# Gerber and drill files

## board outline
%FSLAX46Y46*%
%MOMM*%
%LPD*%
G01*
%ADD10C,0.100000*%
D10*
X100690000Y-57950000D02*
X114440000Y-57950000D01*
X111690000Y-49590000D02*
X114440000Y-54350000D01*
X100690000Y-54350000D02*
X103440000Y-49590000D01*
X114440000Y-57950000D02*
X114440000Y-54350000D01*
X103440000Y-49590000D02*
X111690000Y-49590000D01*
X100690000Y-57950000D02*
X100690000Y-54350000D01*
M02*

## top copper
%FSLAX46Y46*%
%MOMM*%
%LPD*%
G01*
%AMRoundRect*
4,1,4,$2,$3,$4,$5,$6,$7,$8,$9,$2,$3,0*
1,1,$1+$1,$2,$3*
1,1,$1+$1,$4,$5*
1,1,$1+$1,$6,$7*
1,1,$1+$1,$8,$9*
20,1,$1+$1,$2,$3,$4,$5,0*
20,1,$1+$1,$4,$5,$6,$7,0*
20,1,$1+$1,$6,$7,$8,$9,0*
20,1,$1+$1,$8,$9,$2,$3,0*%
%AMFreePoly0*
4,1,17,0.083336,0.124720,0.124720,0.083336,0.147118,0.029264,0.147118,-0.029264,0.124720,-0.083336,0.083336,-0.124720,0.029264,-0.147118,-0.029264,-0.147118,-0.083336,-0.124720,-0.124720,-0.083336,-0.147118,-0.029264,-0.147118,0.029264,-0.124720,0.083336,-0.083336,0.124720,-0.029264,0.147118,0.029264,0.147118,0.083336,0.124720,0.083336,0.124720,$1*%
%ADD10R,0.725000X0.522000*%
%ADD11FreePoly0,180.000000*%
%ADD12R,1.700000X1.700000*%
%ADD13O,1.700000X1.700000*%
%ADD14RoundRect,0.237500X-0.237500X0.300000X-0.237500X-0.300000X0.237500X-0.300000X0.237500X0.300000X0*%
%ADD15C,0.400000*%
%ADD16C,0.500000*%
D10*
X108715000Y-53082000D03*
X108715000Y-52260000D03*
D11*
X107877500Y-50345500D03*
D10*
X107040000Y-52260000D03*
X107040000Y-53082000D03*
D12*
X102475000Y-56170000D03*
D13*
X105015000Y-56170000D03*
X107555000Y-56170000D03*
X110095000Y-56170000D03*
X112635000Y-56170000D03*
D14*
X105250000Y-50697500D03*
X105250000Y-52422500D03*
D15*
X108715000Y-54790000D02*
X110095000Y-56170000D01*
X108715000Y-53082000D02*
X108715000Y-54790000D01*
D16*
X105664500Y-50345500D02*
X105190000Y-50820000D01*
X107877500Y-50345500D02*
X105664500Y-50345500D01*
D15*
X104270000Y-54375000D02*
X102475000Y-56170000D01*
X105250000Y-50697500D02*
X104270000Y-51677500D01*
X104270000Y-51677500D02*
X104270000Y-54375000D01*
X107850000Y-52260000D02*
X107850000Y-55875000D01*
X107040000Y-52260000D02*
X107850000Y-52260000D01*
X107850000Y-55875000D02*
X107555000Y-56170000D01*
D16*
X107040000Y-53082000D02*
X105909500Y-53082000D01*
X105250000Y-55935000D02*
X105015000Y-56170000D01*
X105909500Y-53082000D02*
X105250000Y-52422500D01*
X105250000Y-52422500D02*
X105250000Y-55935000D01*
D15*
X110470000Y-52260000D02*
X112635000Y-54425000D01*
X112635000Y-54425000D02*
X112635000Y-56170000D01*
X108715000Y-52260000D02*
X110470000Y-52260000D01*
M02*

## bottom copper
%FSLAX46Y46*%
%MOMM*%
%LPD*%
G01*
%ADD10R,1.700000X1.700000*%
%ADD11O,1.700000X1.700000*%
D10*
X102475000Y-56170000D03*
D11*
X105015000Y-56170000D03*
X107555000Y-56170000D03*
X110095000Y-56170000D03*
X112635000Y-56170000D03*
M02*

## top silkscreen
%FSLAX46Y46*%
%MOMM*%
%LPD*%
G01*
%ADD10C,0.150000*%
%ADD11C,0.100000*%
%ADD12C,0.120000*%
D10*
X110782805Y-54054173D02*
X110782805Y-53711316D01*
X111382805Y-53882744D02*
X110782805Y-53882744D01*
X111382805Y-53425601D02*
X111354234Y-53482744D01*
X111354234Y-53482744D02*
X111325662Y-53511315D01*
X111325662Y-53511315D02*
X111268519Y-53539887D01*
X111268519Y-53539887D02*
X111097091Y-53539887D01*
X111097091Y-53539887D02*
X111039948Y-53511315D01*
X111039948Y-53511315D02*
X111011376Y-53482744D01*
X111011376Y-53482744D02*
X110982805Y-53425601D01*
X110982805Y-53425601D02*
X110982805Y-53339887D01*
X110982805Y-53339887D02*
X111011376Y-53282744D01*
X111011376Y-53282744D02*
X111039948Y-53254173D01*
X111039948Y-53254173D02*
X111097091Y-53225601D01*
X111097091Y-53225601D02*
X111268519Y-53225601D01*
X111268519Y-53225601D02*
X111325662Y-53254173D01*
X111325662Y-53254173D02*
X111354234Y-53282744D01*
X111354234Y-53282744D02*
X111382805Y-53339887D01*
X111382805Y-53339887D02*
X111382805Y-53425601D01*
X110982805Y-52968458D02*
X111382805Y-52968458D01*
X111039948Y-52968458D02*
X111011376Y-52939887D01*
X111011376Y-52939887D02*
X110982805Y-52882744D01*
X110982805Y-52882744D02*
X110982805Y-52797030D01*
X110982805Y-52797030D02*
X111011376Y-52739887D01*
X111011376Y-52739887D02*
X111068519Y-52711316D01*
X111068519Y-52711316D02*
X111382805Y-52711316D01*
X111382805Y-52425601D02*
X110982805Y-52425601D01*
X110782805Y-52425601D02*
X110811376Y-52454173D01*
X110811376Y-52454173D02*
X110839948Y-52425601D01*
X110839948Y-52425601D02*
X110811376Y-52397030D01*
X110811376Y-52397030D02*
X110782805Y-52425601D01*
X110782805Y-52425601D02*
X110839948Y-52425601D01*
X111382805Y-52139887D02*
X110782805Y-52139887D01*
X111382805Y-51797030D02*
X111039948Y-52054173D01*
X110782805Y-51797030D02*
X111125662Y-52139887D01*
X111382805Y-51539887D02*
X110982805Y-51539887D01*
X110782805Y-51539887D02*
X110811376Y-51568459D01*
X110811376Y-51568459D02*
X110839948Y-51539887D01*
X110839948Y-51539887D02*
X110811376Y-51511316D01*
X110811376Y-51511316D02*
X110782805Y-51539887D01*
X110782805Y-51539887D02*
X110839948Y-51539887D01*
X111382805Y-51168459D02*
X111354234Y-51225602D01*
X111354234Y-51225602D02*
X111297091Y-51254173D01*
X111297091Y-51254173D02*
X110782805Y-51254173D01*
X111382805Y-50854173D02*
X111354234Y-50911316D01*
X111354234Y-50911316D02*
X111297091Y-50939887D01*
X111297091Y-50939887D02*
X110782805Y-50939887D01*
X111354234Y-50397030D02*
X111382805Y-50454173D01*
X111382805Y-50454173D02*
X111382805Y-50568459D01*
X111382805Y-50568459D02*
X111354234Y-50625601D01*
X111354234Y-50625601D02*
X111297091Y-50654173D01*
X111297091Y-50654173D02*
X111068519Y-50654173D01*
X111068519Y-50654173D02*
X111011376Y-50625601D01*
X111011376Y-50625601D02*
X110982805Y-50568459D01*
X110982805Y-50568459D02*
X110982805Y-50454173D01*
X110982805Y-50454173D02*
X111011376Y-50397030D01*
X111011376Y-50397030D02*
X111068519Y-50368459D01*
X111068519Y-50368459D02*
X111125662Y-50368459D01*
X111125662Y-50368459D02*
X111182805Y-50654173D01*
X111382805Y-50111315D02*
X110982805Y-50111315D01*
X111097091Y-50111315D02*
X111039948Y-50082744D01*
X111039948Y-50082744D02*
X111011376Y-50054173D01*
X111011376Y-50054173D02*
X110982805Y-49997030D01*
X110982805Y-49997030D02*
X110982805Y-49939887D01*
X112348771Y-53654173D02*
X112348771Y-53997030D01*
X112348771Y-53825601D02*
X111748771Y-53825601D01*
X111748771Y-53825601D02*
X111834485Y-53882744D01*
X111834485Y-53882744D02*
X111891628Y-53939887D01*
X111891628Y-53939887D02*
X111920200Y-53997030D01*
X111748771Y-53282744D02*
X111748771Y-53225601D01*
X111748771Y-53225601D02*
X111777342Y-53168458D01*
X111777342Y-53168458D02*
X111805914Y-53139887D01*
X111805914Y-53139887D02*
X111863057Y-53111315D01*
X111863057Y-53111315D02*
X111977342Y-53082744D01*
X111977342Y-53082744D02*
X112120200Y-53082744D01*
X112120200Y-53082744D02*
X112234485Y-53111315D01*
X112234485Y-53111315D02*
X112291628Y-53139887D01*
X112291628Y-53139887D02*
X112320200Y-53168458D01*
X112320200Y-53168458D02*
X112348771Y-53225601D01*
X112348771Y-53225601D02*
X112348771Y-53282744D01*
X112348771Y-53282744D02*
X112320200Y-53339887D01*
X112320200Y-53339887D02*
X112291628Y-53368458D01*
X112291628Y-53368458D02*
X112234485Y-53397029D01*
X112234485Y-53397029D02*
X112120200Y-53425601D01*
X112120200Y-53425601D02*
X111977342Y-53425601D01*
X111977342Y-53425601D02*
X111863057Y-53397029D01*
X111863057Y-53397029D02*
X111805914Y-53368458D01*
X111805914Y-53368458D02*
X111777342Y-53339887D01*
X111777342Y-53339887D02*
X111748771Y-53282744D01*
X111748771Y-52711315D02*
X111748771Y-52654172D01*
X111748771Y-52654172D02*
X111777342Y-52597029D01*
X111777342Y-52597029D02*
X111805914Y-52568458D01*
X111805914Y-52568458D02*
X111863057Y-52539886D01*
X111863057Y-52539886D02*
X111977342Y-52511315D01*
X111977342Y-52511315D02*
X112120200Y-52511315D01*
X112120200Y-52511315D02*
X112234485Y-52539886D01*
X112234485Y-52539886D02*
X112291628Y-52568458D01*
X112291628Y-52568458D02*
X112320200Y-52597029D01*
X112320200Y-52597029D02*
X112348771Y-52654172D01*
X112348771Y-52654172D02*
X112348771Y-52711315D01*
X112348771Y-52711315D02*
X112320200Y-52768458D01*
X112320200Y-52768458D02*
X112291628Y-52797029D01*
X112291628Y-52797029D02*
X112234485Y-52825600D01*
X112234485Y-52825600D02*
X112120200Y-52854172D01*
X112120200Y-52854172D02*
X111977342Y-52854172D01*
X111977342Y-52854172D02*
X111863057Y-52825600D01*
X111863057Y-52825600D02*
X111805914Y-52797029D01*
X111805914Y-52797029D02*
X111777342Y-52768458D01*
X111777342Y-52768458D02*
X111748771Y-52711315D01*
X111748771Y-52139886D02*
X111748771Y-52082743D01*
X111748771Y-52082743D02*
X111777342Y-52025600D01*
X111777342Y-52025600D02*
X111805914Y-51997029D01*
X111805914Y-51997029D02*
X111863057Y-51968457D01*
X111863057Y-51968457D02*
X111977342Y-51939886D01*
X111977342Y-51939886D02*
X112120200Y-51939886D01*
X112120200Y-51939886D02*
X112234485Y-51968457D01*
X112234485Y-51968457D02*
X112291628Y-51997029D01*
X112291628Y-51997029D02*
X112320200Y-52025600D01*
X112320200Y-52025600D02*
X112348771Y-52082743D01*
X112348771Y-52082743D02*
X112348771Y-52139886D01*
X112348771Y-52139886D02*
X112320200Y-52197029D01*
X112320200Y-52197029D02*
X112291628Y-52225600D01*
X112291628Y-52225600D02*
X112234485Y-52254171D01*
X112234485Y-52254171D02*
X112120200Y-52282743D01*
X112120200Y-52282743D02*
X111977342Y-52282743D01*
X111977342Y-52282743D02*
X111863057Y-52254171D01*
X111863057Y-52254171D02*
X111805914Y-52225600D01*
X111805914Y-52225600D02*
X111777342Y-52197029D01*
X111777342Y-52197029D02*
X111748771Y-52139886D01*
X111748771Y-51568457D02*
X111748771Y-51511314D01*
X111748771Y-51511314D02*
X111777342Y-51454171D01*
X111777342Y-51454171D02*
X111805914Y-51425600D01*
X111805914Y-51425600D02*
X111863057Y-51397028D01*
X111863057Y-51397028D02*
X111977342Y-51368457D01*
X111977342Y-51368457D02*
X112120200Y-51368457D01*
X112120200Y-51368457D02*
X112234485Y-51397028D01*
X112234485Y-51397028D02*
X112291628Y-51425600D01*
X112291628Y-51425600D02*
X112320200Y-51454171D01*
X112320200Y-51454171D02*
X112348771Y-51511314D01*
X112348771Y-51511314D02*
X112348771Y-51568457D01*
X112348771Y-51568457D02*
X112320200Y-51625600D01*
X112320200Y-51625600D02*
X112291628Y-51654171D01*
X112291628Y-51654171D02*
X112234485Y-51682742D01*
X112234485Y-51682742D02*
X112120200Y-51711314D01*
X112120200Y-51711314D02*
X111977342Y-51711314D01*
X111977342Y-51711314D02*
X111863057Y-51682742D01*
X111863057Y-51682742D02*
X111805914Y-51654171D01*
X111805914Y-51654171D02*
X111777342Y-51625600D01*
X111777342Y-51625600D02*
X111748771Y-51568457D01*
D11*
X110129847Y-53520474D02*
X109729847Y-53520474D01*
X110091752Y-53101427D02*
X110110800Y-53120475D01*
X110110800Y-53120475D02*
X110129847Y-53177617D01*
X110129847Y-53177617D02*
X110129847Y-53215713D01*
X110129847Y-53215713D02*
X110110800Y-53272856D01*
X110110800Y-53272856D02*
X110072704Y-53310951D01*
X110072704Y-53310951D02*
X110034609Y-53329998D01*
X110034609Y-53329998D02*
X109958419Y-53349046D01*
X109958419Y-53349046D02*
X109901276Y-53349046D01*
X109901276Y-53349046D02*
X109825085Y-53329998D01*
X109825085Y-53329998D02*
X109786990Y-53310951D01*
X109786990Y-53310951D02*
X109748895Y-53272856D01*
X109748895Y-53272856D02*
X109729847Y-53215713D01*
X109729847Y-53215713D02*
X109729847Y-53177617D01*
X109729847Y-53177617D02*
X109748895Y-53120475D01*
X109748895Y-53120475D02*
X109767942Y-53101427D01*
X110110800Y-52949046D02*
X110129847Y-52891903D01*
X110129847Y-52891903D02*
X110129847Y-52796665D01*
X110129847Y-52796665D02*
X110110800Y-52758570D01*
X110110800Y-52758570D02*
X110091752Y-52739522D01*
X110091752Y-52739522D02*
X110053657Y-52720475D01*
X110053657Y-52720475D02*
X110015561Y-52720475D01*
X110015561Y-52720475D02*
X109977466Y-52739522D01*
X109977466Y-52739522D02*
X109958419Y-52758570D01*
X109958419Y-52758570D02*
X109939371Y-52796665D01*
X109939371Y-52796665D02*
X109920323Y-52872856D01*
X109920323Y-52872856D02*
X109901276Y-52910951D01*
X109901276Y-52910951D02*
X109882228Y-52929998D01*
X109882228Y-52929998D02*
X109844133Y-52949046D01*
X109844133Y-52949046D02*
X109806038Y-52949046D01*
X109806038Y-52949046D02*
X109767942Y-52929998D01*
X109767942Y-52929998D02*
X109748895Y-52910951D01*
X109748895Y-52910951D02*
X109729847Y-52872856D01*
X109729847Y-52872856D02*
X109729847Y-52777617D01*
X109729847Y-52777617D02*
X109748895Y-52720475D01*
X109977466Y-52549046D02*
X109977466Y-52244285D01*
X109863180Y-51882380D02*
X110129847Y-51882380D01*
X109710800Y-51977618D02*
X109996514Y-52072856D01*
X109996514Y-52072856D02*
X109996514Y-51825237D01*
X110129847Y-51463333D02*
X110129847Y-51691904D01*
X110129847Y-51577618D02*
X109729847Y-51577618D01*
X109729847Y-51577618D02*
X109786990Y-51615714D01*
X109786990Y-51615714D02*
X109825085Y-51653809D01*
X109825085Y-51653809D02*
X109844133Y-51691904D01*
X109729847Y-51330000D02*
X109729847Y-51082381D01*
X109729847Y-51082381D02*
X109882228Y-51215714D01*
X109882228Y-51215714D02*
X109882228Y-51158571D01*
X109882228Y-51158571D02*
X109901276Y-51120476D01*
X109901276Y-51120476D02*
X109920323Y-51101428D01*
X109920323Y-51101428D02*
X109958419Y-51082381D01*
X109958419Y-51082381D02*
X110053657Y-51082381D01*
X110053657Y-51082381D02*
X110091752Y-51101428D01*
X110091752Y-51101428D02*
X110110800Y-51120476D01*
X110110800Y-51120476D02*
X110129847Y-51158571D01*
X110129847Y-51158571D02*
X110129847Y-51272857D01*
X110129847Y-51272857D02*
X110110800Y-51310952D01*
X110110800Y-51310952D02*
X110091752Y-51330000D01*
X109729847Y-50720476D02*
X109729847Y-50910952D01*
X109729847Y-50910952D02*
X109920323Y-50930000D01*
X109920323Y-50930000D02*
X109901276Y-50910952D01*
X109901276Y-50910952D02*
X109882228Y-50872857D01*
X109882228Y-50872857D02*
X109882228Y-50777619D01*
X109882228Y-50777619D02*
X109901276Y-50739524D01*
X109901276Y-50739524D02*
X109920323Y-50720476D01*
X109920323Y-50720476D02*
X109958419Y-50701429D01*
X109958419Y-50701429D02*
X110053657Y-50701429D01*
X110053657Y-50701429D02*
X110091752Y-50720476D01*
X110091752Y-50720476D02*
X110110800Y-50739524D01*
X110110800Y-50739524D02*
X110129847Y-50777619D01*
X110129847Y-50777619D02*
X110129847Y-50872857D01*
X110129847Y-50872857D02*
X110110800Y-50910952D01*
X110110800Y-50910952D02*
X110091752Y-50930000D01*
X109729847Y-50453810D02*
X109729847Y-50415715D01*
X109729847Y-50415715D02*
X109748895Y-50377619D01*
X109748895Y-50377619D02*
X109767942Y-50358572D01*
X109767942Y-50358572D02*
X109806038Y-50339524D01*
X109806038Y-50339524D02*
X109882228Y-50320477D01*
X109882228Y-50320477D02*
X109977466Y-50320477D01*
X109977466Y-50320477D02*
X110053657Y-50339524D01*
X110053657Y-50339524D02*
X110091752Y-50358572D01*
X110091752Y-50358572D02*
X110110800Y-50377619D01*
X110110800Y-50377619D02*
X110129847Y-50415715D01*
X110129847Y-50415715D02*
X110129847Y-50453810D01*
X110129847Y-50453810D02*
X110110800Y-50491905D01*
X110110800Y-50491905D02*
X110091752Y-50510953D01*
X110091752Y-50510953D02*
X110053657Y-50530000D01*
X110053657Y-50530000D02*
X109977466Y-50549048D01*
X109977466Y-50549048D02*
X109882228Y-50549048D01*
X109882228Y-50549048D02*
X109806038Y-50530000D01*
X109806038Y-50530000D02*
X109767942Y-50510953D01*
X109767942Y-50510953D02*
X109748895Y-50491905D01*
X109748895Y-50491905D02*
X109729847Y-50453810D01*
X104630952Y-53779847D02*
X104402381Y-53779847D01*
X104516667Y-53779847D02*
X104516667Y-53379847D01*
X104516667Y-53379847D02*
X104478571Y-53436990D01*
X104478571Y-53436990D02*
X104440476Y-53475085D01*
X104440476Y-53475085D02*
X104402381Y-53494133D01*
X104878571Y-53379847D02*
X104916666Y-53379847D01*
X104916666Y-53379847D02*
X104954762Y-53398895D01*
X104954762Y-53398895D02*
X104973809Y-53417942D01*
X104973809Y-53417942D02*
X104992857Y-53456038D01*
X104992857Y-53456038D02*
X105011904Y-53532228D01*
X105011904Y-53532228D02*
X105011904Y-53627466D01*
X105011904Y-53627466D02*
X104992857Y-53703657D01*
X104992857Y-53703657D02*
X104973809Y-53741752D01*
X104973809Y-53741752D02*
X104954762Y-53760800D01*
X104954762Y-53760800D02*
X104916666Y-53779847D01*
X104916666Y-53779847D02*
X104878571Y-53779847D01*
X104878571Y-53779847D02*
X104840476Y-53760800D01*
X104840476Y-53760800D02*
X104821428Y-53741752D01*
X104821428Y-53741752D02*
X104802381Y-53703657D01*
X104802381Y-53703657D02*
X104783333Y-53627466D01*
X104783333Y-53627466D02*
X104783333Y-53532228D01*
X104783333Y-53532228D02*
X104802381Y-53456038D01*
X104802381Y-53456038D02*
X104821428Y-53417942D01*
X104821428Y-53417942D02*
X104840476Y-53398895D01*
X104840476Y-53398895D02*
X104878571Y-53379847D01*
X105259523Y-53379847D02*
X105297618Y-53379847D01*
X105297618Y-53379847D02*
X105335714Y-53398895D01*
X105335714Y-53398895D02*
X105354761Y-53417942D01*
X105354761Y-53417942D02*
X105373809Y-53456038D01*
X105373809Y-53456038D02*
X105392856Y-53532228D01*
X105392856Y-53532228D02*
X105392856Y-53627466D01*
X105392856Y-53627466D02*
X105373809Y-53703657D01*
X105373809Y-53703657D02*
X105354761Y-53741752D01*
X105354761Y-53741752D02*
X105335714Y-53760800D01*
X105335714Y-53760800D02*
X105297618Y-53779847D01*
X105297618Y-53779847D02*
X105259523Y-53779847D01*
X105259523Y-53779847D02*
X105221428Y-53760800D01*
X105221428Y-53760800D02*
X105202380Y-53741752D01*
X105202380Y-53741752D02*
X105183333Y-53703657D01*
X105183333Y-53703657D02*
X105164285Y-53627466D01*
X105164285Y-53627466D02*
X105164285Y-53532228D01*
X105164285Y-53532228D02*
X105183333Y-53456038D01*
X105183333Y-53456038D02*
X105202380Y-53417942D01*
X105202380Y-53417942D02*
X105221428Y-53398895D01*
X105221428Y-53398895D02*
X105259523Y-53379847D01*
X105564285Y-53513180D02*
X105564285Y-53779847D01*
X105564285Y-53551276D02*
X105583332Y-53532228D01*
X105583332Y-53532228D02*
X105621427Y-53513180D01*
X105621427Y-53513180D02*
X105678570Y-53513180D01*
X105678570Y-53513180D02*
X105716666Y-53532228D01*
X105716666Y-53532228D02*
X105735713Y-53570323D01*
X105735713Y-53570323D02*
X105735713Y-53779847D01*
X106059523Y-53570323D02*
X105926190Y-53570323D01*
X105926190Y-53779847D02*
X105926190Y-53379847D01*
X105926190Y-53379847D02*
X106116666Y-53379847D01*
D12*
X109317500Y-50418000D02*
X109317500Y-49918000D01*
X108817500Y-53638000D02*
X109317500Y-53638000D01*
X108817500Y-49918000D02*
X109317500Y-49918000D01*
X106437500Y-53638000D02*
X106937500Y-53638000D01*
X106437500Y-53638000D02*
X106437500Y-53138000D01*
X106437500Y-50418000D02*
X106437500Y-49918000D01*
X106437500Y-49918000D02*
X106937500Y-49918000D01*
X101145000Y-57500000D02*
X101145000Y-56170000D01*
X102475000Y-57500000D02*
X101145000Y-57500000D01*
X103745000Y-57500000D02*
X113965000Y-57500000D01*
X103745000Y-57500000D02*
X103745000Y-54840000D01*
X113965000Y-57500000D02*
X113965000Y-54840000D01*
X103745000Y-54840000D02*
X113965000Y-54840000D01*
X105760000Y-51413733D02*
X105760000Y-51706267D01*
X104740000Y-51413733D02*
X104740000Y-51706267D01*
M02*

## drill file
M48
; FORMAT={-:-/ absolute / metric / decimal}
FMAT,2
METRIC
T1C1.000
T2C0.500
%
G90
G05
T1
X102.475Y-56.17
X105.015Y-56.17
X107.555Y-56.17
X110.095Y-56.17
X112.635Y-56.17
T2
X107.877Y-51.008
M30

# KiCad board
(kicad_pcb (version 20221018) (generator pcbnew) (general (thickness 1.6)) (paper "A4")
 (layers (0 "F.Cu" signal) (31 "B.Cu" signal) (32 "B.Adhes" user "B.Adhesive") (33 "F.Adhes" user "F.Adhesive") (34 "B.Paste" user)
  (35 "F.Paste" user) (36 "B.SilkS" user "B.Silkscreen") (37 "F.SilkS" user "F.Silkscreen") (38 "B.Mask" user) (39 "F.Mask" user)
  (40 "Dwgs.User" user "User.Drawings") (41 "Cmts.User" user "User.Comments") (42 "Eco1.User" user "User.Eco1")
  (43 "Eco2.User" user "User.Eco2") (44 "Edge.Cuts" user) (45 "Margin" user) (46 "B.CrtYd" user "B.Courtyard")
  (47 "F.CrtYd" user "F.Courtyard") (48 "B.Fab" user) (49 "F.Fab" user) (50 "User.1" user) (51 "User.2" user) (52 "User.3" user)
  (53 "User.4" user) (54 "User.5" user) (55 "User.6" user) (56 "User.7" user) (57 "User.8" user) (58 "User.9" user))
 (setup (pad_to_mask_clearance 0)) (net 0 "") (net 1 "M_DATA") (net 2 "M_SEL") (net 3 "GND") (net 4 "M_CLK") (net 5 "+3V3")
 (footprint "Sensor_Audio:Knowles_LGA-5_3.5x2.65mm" (layer "F.Cu") (at 107.8775 51.778 180)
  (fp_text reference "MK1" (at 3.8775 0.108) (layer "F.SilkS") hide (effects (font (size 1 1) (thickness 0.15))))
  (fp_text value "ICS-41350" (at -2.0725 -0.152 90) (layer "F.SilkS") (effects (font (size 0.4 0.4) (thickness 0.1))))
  (fp_line (start -1.44 1.36) (end -1.44 1.86) (stroke (width 0.12) (type solid)) (layer "F.SilkS"))
  (fp_line (start -0.94 -1.86) (end -1.44 -1.86) (stroke (width 0.12) (type solid)) (layer "F.SilkS"))
  (fp_line (start -0.94 1.86) (end -1.44 1.86) (stroke (width 0.12) (type solid)) (layer "F.SilkS"))
  (fp_line (start 1.44 -1.86) (end 0.94 -1.86) (stroke (width 0.12) (type solid)) (layer "F.SilkS"))
  (fp_line (start 1.44 -1.86) (end 1.44 -1.36) (stroke (width 0.12) (type solid)) (layer "F.SilkS"))
  (fp_line (start 1.44 1.36) (end 1.44 1.86) (stroke (width 0.12) (type solid)) (layer "F.SilkS"))
  (fp_line (start 1.44 1.86) (end 0.94 1.86) (stroke (width 0.12) (type solid)) (layer "F.SilkS"))
  (pad "" np_thru_hole circle (at 0 0.77 180) (size 0.5 0.5) (drill 0.5) (layers "F&B.Cu" "*.Mask"))
  (pad "1" smd rect (at -0.8375 -1.304 180) (size 0.725 0.522) (layers "F.Cu" "F.Paste" "F.Mask") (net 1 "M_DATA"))
  (pad "2" smd rect (at -0.8375 -0.482 180) (size 0.725 0.522) (layers "F.Cu" "F.Paste" "F.Mask") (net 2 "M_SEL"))
  (pad "3" smd custom (at 0 1.4325 180) (size 0.3 0.3) (layers "F.Cu" "F.Mask") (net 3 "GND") (zone_connect 0) (thermal_bridge_angle 90)
   (options (clearance outline) (anchor circle)) (primitives))
  (pad "4" smd rect (at 0.8375 -0.482 180) (size 0.725 0.522) (layers "F.Cu" "F.Paste" "F.Mask") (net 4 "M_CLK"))
  (pad "5" smd rect (at 0.8375 -1.304 180) (size 0.725 0.522) (layers "F.Cu" "F.Paste" "F.Mask") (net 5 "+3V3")))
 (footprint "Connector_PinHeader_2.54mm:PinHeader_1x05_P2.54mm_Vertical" (layer "F.Cu") (at 102.475 56.17 90)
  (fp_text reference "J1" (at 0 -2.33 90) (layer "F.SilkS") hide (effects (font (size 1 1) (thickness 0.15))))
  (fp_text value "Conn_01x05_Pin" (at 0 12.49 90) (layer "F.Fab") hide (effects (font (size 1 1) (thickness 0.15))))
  (fp_line (start -1.33 -1.33) (end 0 -1.33) (stroke (width 0.12) (type solid)) (layer "F.SilkS"))
  (fp_line (start -1.33 0) (end -1.33 -1.33) (stroke (width 0.12) (type solid)) (layer "F.SilkS"))
  (fp_line (start -1.33 1.27) (end -1.33 11.49) (stroke (width 0.12) (type solid)) (layer "F.SilkS"))
  (fp_line (start -1.33 1.27) (end 1.33 1.27) (stroke (width 0.12) (type solid)) (layer "F.SilkS"))
  (fp_line (start -1.33 11.49) (end 1.33 11.49) (stroke (width 0.12) (type solid)) (layer "F.SilkS"))
  (fp_line (start 1.33 1.27) (end 1.33 11.49) (stroke (width 0.12) (type solid)) (layer "F.SilkS"))
  (pad "1" thru_hole rect (at 0 0 90) (size 1.7 1.7) (drill 1) (layers "*.Cu" "*.Mask") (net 3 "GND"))
  (pad "2" thru_hole oval (at 0 2.54 90) (size 1.7 1.7) (drill 1) (layers "*.Cu" "*.Mask") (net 5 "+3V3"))
  (pad "3" thru_hole oval (at 0 5.08 90) (size 1.7 1.7) (drill 1) (layers "*.Cu" "*.Mask") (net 4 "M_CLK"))
  (pad "4" thru_hole oval (at 0 7.62 90) (size 1.7 1.7) (drill 1) (layers "*.Cu" "*.Mask") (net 1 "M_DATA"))
  (pad "5" thru_hole oval (at 0 10.16 90) (size 1.7 1.7) (drill 1) (layers "*.Cu" "*.Mask") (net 2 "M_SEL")))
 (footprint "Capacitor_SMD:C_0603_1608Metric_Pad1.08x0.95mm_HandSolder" (layer "F.Cu") (at 105.25 51.56 -90)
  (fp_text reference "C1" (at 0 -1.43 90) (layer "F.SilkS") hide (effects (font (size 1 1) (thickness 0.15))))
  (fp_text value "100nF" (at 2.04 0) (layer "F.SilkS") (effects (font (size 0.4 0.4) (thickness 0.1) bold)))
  (fp_line (start -0.146267 -0.51) (end 0.146267 -0.51) (stroke (width 0.12) (type solid)) (layer "F.SilkS"))
  (fp_line (start -0.146267 0.51) (end 0.146267 0.51) (stroke (width 0.12) (type solid)) (layer "F.SilkS"))
  (pad "1" smd roundrect (at -0.8625 0 270) (size 1.075 0.95) (layers "F.Cu" "F.Paste" "F.Mask") (roundrect_rratio 0.25) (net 3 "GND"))
  (pad "2" smd roundrect (at 0.8625 0 270) (size 1.075 0.95) (layers "F.Cu" "F.Paste" "F.Mask") (roundrect_rratio 0.25) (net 5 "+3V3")))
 (gr_line (start 100.69 57.95) (end 114.44 57.95) (stroke (width 0.1) (type default)) (layer "Edge.Cuts"))
 (gr_line (start 111.69 49.59) (end 114.44 54.35) (stroke (width 0.1) (type default)) (layer "Edge.Cuts"))
 (gr_line (start 100.69 54.35) (end 103.44 49.59) (stroke (width 0.1) (type default)) (layer "Edge.Cuts"))
 (gr_line (start 114.44 57.95) (end 114.44 54.35) (stroke (width 0.1) (type default)) (layer "Edge.Cuts"))
 (gr_line (start 103.44 49.59) (end 111.69 49.59) (stroke (width 0.1) (type default)) (layer "Edge.Cuts"))
 (gr_line (start 100.69 57.95) (end 100.69 54.35) (stroke (width 0.1) (type default)) (layer "Edge.Cuts"))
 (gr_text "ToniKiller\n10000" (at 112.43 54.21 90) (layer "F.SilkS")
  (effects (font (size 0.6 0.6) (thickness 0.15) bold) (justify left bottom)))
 (segment (start 108.715 54.79) (end 110.095 56.17) (width 0.4) (layer "F.Cu") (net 1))
 (segment (start 108.715 53.082) (end 108.715 54.79) (width 0.4) (layer "F.Cu") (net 1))
 (segment (start 105.6645 50.3455) (end 105.19 50.82) (width 0.5) (layer "F.Cu") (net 3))
 (segment (start 107.8775 50.3455) (end 105.6645 50.3455) (width 0.5) (layer "F.Cu") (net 3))
 (segment (start 104.27 54.375) (end 102.475 56.17) (width 0.4) (layer "F.Cu") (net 3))
 (segment (start 105.25 50.6975) (end 104.27 51.6775) (width 0.4) (layer "F.Cu") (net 3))
 (segment (start 104.27 51.6775) (end 104.27 54.375) (width 0.4) (layer "F.Cu") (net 3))
 (segment (start 107.85 52.26) (end 107.85 55.875) (width 0.4) (layer "F.Cu") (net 4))
 (segment (start 107.04 52.26) (end 107.85 52.26) (width 0.4) (layer "F.Cu") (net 4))
 (segment (start 107.85 55.875) (end 107.555 56.17) (width 0.4) (layer "F.Cu") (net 4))
 (segment (start 107.04 53.082) (end 105.9095 53.082) (width 0.5) (layer "F.Cu") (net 5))
 (segment (start 105.25 55.935) (end 105.015 56.17) (width 0.5) (layer "F.Cu") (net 5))
 (segment (start 105.9095 53.082) (end 105.25 52.4225) (width 0.5) (layer "F.Cu") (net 5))
 (segment (start 105.25 52.4225) (end 105.25 55.935) (width 0.5) (layer "F.Cu") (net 5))
 (segment (start 110.47 52.26) (end 112.635 54.425) (width 0.4) (layer "F.Cu") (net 2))
 (segment (start 112.635 54.425) (end 112.635 56.17) (width 0.4) (layer "F.Cu") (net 2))
 (segment (start 108.715 52.26) (end 110.47 52.26) (width 0.4) (layer "F.Cu") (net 2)))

